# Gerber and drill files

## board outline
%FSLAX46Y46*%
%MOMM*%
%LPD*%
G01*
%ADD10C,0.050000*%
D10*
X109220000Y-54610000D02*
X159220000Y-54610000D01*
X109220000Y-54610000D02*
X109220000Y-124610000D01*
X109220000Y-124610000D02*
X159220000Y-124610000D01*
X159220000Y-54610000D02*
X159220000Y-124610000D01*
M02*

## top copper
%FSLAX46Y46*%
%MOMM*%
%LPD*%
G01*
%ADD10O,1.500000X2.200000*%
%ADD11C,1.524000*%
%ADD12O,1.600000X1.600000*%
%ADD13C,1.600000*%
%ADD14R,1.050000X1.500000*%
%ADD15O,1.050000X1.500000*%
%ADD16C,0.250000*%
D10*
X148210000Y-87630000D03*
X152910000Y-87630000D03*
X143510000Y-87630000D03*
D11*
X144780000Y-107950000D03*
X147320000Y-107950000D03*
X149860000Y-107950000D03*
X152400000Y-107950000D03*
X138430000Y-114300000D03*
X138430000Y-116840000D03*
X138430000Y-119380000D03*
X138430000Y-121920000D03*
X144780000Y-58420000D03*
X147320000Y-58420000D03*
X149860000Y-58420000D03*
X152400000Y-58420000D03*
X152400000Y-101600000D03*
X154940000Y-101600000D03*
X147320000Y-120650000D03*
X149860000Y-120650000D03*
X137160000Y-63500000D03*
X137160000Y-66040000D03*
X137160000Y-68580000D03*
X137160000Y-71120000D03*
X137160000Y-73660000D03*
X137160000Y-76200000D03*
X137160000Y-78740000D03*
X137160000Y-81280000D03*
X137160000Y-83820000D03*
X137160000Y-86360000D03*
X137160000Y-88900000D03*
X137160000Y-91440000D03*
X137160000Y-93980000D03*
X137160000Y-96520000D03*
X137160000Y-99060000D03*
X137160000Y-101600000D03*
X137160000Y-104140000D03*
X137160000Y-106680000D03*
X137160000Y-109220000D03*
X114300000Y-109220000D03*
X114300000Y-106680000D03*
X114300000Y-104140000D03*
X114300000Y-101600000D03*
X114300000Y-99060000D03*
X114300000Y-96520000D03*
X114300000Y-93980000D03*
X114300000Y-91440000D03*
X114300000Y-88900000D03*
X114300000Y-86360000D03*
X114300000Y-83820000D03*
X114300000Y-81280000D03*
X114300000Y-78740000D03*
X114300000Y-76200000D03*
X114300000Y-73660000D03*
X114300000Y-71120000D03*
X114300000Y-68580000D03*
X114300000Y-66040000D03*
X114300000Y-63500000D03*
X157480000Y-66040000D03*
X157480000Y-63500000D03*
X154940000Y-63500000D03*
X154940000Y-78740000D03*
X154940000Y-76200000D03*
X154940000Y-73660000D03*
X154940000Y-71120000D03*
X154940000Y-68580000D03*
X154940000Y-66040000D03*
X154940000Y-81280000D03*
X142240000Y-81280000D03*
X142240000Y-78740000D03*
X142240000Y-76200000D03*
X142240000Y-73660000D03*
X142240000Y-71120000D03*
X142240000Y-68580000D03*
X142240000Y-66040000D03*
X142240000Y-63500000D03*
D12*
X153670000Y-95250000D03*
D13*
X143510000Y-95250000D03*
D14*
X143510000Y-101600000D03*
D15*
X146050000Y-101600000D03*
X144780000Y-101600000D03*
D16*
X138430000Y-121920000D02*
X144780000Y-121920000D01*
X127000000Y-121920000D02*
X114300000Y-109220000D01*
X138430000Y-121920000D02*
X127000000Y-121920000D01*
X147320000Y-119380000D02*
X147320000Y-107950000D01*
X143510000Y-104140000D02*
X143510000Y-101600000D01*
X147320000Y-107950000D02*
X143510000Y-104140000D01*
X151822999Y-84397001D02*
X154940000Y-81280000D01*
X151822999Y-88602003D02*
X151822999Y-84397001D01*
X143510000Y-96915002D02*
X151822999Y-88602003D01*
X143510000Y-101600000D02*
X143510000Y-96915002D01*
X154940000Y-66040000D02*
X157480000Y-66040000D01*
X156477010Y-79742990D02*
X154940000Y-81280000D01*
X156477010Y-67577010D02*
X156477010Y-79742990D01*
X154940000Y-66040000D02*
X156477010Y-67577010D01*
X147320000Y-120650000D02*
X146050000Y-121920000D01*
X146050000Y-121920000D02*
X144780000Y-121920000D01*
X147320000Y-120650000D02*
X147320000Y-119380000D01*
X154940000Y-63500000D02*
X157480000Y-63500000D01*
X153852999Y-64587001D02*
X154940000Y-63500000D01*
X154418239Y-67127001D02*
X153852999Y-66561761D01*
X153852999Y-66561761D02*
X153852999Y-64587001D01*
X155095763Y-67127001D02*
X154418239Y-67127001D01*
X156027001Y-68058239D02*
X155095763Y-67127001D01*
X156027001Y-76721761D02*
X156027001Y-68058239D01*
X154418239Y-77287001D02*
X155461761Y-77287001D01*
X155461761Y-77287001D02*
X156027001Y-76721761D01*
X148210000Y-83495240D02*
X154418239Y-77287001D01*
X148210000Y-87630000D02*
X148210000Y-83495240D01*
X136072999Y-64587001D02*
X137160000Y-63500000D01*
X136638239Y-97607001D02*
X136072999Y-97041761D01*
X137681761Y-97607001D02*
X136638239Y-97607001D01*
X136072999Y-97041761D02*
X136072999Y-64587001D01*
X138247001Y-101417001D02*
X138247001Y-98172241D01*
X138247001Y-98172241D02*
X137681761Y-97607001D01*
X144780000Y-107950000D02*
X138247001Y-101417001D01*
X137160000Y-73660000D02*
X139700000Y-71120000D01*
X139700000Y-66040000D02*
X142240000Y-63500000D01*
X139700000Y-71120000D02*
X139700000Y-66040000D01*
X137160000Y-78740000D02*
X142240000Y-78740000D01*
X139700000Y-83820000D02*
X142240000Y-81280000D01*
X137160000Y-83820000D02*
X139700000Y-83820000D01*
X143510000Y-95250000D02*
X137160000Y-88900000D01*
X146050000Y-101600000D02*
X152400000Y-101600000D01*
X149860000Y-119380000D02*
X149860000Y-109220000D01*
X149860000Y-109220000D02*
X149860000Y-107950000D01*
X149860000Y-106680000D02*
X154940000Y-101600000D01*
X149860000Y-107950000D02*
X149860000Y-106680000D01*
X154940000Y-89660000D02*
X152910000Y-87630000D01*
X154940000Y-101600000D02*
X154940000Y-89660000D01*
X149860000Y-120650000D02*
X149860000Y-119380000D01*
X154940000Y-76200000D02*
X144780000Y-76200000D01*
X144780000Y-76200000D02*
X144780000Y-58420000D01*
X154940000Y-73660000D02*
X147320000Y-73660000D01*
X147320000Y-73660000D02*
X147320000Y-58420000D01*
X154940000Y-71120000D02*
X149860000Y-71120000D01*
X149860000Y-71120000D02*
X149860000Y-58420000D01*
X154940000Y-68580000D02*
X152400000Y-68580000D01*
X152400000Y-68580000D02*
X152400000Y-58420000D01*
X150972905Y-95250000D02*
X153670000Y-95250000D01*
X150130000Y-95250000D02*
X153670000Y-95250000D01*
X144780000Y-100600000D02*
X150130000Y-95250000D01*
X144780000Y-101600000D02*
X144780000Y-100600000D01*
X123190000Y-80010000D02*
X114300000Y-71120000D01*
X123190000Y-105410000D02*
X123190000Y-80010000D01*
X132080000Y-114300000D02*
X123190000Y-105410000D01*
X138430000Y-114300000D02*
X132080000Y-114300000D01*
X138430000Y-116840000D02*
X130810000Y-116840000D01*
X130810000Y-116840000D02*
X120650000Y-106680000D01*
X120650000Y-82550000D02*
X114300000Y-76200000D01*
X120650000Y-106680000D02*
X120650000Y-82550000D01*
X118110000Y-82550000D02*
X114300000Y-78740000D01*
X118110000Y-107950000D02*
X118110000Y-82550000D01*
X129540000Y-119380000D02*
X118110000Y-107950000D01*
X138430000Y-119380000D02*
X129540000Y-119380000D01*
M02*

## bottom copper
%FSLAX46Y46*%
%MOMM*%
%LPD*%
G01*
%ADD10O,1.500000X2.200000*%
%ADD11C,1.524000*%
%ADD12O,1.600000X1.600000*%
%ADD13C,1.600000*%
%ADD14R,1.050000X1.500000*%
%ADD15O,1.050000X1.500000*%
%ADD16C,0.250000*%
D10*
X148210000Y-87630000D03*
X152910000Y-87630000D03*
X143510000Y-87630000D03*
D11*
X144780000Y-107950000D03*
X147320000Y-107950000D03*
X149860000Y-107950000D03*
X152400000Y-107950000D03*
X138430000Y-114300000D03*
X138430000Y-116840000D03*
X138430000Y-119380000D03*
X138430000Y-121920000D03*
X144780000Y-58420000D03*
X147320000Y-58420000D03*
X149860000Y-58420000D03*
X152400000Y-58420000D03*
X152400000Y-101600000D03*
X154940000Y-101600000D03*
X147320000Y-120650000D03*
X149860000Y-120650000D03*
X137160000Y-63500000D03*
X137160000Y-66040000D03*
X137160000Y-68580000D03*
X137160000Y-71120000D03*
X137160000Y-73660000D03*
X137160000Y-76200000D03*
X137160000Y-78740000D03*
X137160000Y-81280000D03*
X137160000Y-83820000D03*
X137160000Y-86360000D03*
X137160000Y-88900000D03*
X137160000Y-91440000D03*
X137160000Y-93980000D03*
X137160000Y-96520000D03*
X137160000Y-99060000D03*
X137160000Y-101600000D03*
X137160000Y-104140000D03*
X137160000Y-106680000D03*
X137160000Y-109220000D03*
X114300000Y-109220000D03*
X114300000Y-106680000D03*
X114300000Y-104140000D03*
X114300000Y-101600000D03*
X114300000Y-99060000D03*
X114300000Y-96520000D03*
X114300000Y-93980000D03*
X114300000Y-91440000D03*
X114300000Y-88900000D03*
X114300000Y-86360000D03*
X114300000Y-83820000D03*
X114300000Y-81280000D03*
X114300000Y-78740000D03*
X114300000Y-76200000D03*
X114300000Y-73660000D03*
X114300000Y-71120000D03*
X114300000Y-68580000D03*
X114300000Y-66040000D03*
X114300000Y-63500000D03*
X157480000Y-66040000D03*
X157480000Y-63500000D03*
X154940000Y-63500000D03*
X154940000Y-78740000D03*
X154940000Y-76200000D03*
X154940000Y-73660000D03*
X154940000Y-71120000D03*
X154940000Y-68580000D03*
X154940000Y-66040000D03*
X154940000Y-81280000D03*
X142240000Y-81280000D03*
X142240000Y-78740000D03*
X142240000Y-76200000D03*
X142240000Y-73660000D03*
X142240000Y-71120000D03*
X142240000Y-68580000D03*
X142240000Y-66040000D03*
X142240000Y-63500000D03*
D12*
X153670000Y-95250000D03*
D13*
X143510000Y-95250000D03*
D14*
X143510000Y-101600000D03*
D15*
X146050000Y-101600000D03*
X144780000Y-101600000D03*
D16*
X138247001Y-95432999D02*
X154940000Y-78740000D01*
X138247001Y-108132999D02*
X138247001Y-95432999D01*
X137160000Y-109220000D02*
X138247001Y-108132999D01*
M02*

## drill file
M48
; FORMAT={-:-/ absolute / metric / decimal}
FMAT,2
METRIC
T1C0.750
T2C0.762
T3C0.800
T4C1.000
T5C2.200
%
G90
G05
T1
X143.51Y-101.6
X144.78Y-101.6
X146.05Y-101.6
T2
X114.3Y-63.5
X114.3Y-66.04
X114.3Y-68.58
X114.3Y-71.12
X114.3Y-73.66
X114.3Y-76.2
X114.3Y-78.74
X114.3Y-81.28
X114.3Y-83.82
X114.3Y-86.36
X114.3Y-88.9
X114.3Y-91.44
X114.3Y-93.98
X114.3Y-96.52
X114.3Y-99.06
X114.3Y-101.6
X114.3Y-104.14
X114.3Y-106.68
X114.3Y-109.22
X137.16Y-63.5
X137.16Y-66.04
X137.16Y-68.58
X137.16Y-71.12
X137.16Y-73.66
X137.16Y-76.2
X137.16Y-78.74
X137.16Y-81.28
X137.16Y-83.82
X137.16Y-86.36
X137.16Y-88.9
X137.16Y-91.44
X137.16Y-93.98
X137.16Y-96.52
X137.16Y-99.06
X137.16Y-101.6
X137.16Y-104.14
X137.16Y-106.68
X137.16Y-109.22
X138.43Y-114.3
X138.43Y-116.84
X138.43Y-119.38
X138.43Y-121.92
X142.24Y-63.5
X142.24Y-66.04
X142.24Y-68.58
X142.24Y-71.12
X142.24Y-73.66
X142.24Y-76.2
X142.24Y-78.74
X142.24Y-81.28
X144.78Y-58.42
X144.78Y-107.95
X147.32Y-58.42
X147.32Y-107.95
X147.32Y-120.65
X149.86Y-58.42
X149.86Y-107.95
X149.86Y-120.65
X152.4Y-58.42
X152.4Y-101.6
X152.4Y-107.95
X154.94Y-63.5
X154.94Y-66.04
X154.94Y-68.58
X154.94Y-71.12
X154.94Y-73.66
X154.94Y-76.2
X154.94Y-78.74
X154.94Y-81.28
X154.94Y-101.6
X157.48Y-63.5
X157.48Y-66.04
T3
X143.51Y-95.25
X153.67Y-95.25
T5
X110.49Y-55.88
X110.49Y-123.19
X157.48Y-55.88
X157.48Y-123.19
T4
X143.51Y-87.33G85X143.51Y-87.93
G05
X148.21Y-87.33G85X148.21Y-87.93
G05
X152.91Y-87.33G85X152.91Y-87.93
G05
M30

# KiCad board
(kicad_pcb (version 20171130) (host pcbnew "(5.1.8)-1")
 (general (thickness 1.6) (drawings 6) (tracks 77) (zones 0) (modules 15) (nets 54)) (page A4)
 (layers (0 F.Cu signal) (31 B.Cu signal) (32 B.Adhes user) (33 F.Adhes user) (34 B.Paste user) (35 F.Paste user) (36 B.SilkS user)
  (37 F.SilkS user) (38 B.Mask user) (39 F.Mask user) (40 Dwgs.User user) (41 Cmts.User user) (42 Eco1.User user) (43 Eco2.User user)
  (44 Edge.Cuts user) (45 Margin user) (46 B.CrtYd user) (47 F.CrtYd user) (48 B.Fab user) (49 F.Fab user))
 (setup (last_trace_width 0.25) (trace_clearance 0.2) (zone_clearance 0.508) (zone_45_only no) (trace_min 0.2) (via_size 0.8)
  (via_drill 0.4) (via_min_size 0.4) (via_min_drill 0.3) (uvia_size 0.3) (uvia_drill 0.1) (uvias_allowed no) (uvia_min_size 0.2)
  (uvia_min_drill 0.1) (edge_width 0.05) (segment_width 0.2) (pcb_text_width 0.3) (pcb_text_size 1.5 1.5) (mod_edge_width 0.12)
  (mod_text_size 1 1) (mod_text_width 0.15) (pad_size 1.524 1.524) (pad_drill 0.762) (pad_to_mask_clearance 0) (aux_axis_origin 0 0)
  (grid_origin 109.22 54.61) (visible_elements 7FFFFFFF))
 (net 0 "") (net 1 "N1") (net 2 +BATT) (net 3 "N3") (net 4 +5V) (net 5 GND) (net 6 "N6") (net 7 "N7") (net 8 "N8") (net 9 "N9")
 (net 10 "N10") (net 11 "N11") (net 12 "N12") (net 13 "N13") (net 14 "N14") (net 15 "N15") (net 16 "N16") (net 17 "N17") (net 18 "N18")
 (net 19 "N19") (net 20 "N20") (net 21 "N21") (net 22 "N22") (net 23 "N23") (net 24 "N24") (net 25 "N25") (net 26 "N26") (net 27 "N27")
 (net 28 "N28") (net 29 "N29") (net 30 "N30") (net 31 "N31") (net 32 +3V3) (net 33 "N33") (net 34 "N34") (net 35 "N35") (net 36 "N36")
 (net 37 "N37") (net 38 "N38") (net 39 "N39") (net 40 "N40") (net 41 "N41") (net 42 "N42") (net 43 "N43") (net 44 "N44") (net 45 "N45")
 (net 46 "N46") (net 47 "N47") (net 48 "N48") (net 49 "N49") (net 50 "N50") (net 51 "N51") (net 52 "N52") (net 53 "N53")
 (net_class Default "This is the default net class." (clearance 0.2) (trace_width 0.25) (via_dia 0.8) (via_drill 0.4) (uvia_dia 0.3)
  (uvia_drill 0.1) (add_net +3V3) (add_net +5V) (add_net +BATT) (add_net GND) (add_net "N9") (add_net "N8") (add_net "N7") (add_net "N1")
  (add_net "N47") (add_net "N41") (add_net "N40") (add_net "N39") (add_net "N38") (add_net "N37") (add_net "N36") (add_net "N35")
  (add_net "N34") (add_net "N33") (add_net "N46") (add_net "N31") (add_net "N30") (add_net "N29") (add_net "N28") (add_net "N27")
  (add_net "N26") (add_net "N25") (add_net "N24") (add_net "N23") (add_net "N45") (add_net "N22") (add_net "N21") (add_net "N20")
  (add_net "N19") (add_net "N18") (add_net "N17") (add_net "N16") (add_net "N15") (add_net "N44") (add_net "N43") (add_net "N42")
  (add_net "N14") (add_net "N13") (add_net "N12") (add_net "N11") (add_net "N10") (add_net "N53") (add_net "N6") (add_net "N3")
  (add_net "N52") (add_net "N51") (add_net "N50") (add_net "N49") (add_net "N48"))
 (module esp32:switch (layer F.Cu) (at 143.51 87.63)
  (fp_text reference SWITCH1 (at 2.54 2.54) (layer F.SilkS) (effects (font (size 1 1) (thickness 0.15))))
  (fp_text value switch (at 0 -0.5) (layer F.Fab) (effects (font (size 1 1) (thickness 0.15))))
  (pad 2 thru_hole oval (at 4.7 0) (size 1.5 2.2) (drill oval 1 1.6) (layers *.Cu *.Mask) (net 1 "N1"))
  (pad 3 thru_hole oval (at 9.4 0) (size 1.5 2.2) (drill oval 1 1.6) (layers *.Cu *.Mask) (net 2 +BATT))
  (pad 1 thru_hole oval (at 0 0) (size 1.5 2.2) (drill oval 1 1.6) (layers *.Cu *.Mask) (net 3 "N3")))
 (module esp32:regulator (layer F.Cu) (at 142.24 105.41)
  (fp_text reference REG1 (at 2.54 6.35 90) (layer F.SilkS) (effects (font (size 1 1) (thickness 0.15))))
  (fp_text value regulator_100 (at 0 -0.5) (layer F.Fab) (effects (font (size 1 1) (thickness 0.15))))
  (pad 1 thru_hole circle (at 2.54 2.54 270) (size 1.524 1.524) (drill 0.762) (layers *.Cu *.Mask) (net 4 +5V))
  (pad 2 thru_hole circle (at 5.08 2.54 270) (size 1.524 1.524) (drill 0.762) (layers *.Cu *.Mask) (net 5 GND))
  (pad 3 thru_hole circle (at 7.62 2.54 270) (size 1.524 1.524) (drill 0.762) (layers *.Cu *.Mask) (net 2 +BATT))
  (pad 4 thru_hole circle (at 10.16 2.54 270) (size 1.524 1.524) (drill 0.762) (layers *.Cu *.Mask) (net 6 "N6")))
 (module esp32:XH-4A (layer F.Cu) (at 138.43 121.92 90)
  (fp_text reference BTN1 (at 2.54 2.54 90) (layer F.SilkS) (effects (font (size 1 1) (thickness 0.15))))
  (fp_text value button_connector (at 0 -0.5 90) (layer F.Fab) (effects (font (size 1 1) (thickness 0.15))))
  (pad 4 thru_hole circle (at 7.62 0 90) (size 1.524 1.524) (drill 0.762) (layers *.Cu *.Mask) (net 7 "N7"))
  (pad 3 thru_hole circle (at 5.08 0 90) (size 1.524 1.524) (drill 0.762) (layers *.Cu *.Mask) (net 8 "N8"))
  (pad 2 thru_hole circle (at 2.54 0 90) (size 1.524 1.524) (drill 0.762) (layers *.Cu *.Mask) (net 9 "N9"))
  (pad 1 thru_hole circle (at 0 0 90) (size 1.524 1.524) (drill 0.762) (layers *.Cu *.Mask) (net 5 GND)))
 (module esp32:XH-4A (layer F.Cu) (at 152.4 58.42 180)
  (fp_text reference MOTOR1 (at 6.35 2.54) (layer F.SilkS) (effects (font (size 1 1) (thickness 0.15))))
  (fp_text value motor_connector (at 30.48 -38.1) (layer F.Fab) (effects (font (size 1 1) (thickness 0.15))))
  (pad 4 thru_hole circle (at 7.62 0 180) (size 1.524 1.524) (drill 0.762) (layers *.Cu *.Mask) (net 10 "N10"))
  (pad 3 thru_hole circle (at 5.08 0 180) (size 1.524 1.524) (drill 0.762) (layers *.Cu *.Mask) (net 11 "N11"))
  (pad 2 thru_hole circle (at 2.54 0 180) (size 1.524 1.524) (drill 0.762) (layers *.Cu *.Mask) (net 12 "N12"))
  (pad 1 thru_hole circle (at 0 0 180) (size 1.524 1.524) (drill 0.762) (layers *.Cu *.Mask) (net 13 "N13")))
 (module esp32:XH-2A (layer F.Cu) (at 154.94 101.6 180)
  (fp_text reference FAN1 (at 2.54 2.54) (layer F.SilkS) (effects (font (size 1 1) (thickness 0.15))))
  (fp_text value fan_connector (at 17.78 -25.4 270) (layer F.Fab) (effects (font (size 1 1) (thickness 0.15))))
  (pad 2 thru_hole circle (at 2.54 0 180) (size 1.524 1.524) (drill 0.762) (layers *.Cu *.Mask) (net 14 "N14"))
  (pad 1 thru_hole circle (at 0 0 180) (size 1.524 1.524) (drill 0.762) (layers *.Cu *.Mask) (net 2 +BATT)))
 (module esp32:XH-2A (layer F.Cu) (at 149.86 120.65 180)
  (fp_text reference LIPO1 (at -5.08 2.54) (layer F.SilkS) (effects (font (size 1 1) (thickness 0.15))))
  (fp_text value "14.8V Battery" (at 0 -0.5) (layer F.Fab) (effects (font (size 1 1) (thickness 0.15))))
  (pad 2 thru_hole circle (at 2.54 0 180) (size 1.524 1.524) (drill 0.762) (layers *.Cu *.Mask) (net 5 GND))
  (pad 1 thru_hole circle (at 0 0 180) (size 1.524 1.524) (drill 0.762) (layers *.Cu *.Mask) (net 2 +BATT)))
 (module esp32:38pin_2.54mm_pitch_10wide (layer F.Cu) (at 111.76 58.42)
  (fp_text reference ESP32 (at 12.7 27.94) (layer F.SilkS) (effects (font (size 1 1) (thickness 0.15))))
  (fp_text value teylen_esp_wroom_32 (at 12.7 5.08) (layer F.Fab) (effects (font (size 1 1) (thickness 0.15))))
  (pad 38 thru_hole circle (at 25.4 5.08) (size 1.524 1.524) (drill 0.762) (layers *.Cu *.Mask) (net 4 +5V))
  (pad 37 thru_hole circle (at 25.4 7.62) (size 1.524 1.524) (drill 0.762) (layers *.Cu *.Mask) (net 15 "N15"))
  (pad 36 thru_hole circle (at 25.4 10.16) (size 1.524 1.524) (drill 0.762) (layers *.Cu *.Mask) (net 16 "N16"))
  (pad 35 thru_hole circle (at 25.4 12.7) (size 1.524 1.524) (drill 0.762) (layers *.Cu *.Mask) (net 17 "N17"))
  (pad 34 thru_hole circle (at 25.4 15.24) (size 1.524 1.524) (drill 0.762) (layers *.Cu *.Mask) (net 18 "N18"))
  (pad 33 thru_hole circle (at 25.4 17.78) (size 1.524 1.524) (drill 0.762) (layers *.Cu *.Mask) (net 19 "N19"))
  (pad 32 thru_hole circle (at 25.4 20.32) (size 1.524 1.524) (drill 0.762) (layers *.Cu *.Mask) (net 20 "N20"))
  (pad 31 thru_hole circle (at 25.4 22.86) (size 1.524 1.524) (drill 0.762) (layers *.Cu *.Mask) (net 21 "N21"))
  (pad 30 thru_hole circle (at 25.4 25.4) (size 1.524 1.524) (drill 0.762) (layers *.Cu *.Mask) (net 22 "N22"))
  (pad 29 thru_hole circle (at 25.4 27.94) (size 1.524 1.524) (drill 0.762) (layers *.Cu *.Mask) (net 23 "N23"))
  (pad 28 thru_hole circle (at 25.4 30.48) (size 1.524 1.524) (drill 0.762) (layers *.Cu *.Mask) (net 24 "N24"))
  (pad 27 thru_hole circle (at 25.4 33.02) (size 1.524 1.524) (drill 0.762) (layers *.Cu *.Mask) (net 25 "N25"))
  (pad 26 thru_hole circle (at 25.4 35.56) (size 1.524 1.524) (drill 0.762) (layers *.Cu *.Mask) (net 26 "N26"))
  (pad 25 thru_hole circle (at 25.4 38.1) (size 1.524 1.524) (drill 0.762) (layers *.Cu *.Mask) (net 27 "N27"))
  (pad 24 thru_hole circle (at 25.4 40.64) (size 1.524 1.524) (drill 0.762) (layers *.Cu *.Mask) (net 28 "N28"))
  (pad 23 thru_hole circle (at 25.4 43.18) (size 1.524 1.524) (drill 0.762) (layers *.Cu *.Mask) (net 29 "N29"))
  (pad 22 thru_hole circle (at 25.4 45.72) (size 1.524 1.524) (drill 0.762) (layers *.Cu *.Mask) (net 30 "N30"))
  (pad 21 thru_hole circle (at 25.4 48.26) (size 1.524 1.524) (drill 0.762) (layers *.Cu *.Mask) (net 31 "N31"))
  (pad 20 thru_hole circle (at 25.4 50.8) (size 1.524 1.524) (drill 0.762) (layers *.Cu *.Mask) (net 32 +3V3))
  (pad 19 thru_hole circle (at 2.54 50.8) (size 1.524 1.524) (drill 0.762) (layers *.Cu *.Mask) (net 5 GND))
  (pad 18 thru_hole circle (at 2.54 48.26) (size 1.524 1.524) (drill 0.762) (layers *.Cu *.Mask) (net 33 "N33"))
  (pad 17 thru_hole circle (at 2.54 45.72) (size 1.524 1.524) (drill 0.762) (layers *.Cu *.Mask) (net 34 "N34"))
  (pad 16 thru_hole circle (at 2.54 43.18) (size 1.524 1.524) (drill 0.762) (layers *.Cu *.Mask) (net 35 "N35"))
  (pad 15 thru_hole circle (at 2.54 40.64) (size 1.524 1.524) (drill 0.762) (layers *.Cu *.Mask) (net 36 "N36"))
  (pad 14 thru_hole circle (at 2.54 38.1) (size 1.524 1.524) (drill 0.762) (layers *.Cu *.Mask) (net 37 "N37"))
  (pad 13 thru_hole circle (at 2.54 35.56) (size 1.524 1.524) (drill 0.762) (layers *.Cu *.Mask) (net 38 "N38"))
  (pad 12 thru_hole circle (at 2.54 33.02) (size 1.524 1.524) (drill 0.762) (layers *.Cu *.Mask) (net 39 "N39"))
  (pad 11 thru_hole circle (at 2.54 30.48) (size 1.524 1.524) (drill 0.762) (layers *.Cu *.Mask) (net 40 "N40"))
  (pad 10 thru_hole circle (at 2.54 27.94) (size 1.524 1.524) (drill 0.762) (layers *.Cu *.Mask) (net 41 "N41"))
  (pad 9 thru_hole circle (at 2.54 25.4) (size 1.524 1.524) (drill 0.762) (layers *.Cu *.Mask) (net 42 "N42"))
  (pad 8 thru_hole circle (at 2.54 22.86) (size 1.524 1.524) (drill 0.762) (layers *.Cu *.Mask) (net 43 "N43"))
  (pad 7 thru_hole circle (at 2.54 20.32) (size 1.524 1.524) (drill 0.762) (layers *.Cu *.Mask) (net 9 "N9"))
  (pad 6 thru_hole circle (at 2.54 17.78) (size 1.524 1.524) (drill 0.762) (layers *.Cu *.Mask) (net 8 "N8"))
  (pad 5 thru_hole circle (at 2.54 15.24) (size 1.524 1.524) (drill 0.762) (layers *.Cu *.Mask) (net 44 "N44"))
  (pad 4 thru_hole circle (at 2.54 12.7) (size 1.524 1.524) (drill 0.762) (layers *.Cu *.Mask) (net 7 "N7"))
  (pad 3 thru_hole circle (at 2.54 10.16) (size 1.524 1.524) (drill 0.762) (layers *.Cu *.Mask) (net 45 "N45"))
  (pad 2 thru_hole circle (at 2.54 7.62) (size 1.524 1.524) (drill 0.762) (layers *.Cu *.Mask) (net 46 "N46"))
  (pad 1 thru_hole circle (at 2.54 5.08) (size 1.524 1.524) (drill 0.762) (layers *.Cu *.Mask) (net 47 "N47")))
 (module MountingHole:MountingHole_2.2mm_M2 (layer F.Cu) (at 157.48 123.19)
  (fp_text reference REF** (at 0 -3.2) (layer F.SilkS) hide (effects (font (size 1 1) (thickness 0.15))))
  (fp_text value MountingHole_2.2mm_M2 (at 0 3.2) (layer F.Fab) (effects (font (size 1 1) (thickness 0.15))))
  (pad 1 np_thru_hole circle (at 0 0) (size 2.2 2.2) (drill 2.2) (layers *.Cu *.Mask)))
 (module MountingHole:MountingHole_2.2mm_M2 (layer F.Cu) (at 110.49 123.19)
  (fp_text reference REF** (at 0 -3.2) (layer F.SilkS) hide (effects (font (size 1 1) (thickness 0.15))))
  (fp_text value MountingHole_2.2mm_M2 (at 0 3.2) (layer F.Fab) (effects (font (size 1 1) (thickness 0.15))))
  (pad 1 np_thru_hole circle (at 0 0) (size 2.2 2.2) (drill 2.2) (layers *.Cu *.Mask)))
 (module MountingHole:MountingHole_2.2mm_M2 (layer F.Cu) (at 157.48 55.88)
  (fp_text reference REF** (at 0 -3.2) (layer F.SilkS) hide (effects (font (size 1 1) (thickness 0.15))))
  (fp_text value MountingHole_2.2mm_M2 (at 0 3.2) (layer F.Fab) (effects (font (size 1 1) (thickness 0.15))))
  (pad 1 np_thru_hole circle (at 0 0) (size 2.2 2.2) (drill 2.2) (layers *.Cu *.Mask)))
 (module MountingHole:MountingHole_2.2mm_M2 (layer F.Cu) (at 110.49 55.88)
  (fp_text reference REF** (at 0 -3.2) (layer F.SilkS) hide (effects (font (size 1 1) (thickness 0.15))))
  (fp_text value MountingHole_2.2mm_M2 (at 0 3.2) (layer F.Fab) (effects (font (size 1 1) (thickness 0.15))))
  (pad 1 np_thru_hole circle (at 0 0) (size 2.2 2.2) (drill 2.2) (layers *.Cu *.Mask)))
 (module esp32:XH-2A (layer F.Cu) (at 162.56 60.96 270)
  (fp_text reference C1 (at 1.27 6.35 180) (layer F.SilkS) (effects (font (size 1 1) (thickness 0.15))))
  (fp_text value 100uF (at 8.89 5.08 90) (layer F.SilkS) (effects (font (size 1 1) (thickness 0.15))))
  (pad 2 thru_hole circle (at 5.08 5.08 270) (size 1.524 1.524) (drill 0.762) (layers *.Cu *.Mask) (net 5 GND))
  (pad 1 thru_hole circle (at 2.54 5.08 270) (size 1.524 1.524) (drill 0.762) (layers *.Cu *.Mask) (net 1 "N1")))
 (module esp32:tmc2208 (layer F.Cu) (at 139.7 60.96)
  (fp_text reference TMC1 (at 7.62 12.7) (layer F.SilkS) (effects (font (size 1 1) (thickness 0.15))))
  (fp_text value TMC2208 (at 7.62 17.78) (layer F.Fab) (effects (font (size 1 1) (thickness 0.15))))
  (pad 16 thru_hole circle (at 15.24 2.54) (size 1.524 1.524) (drill 0.762) (layers *.Cu *.Mask) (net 1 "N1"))
  (pad 10 thru_hole circle (at 15.24 17.78) (size 1.524 1.524) (drill 0.762) (layers *.Cu *.Mask) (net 32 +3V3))
  (pad 11 thru_hole circle (at 15.24 15.24) (size 1.524 1.524) (drill 0.762) (layers *.Cu *.Mask) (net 10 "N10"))
  (pad 12 thru_hole circle (at 15.24 12.7) (size 1.524 1.524) (drill 0.762) (layers *.Cu *.Mask) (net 11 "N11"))
  (pad 13 thru_hole circle (at 15.24 10.16) (size 1.524 1.524) (drill 0.762) (layers *.Cu *.Mask) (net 12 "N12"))
  (pad 14 thru_hole circle (at 15.24 7.62) (size 1.524 1.524) (drill 0.762) (layers *.Cu *.Mask) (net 13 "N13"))
  (pad 15 thru_hole circle (at 15.24 5.08) (size 1.524 1.524) (drill 0.762) (layers *.Cu *.Mask) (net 5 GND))
  (pad 9 thru_hole circle (at 15.24 20.32) (size 1.524 1.524) (drill 0.762) (layers *.Cu *.Mask) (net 5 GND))
  (pad 8 thru_hole circle (at 2.54 20.32) (size 1.524 1.524) (drill 0.762) (layers *.Cu *.Mask) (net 22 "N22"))
  (pad 7 thru_hole circle (at 2.54 17.78) (size 1.524 1.524) (drill 0.762) (layers *.Cu *.Mask) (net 20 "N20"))
  (pad 6 thru_hole circle (at 2.54 15.24) (size 1.524 1.524) (drill 0.762) (layers *.Cu *.Mask) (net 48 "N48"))
  (pad 5 thru_hole circle (at 2.54 12.7) (size 1.524 1.524) (drill 0.762) (layers *.Cu *.Mask) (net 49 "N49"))
  (pad 4 thru_hole circle (at 2.54 10.16) (size 1.524 1.524) (drill 0.762) (layers *.Cu *.Mask) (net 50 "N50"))
  (pad 3 thru_hole circle (at 2.54 7.62) (size 1.524 1.524) (drill 0.762) (layers *.Cu *.Mask) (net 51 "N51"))
  (pad 2 thru_hole circle (at 2.54 5.08) (size 1.524 1.524) (drill 0.762) (layers *.Cu *.Mask) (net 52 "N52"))
  (pad 1 thru_hole circle (at 2.54 2.54) (size 1.524 1.524) (drill 0.762) (layers *.Cu *.Mask) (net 18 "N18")))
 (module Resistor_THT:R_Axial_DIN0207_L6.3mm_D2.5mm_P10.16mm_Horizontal (layer F.Cu) (at 143.51 95.25)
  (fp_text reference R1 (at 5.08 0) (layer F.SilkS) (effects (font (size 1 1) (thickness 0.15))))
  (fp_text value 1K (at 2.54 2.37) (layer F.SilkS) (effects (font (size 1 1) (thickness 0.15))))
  (pad 2 thru_hole oval (at 10.16 0) (size 1.6 1.6) (drill 0.8) (layers *.Cu *.Mask) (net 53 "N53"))
  (pad 1 thru_hole circle (at 0 0) (size 1.6 1.6) (drill 0.8) (layers *.Cu *.Mask) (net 24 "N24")))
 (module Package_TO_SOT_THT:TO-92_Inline (layer F.Cu) (at 143.51 101.6)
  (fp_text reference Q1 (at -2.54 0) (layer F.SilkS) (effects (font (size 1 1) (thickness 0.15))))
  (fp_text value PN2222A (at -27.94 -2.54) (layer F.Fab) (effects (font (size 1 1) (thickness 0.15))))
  (pad 1 thru_hole rect (at 0 0) (size 1.05 1.5) (drill 0.75) (layers *.Cu *.Mask) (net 5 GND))
  (pad 3 thru_hole oval (at 2.54 0) (size 1.05 1.5) (drill 0.75) (layers *.Cu *.Mask) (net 14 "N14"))
  (pad 2 thru_hole oval (at 1.27 0) (size 1.05 1.5) (drill 0.75) (layers *.Cu *.Mask) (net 53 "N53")))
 (gr_line (start 109.22 54.61) (end 159.22 54.61) (layer Edge.Cuts) (width 0.05))
 (gr_line (start 109.22 54.61) (end 109.22 124.61) (layer Edge.Cuts) (width 0.05))
 (gr_line (start 109.22 124.61) (end 159.22 124.61) (layer Edge.Cuts) (width 0.05))
 (gr_line (start 159.22 54.61) (end 159.22 124.61) (layer Edge.Cuts) (width 0.05))
 (segment (start 138.43 121.92) (end 144.78 121.92) (width 0.25) (layer F.Cu) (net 5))
 (segment (start 127 121.92) (end 114.3 109.22) (width 0.25) (layer F.Cu) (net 5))
 (segment (start 138.43 121.92) (end 127 121.92) (width 0.25) (layer F.Cu) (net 5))
 (segment (start 147.32 119.38) (end 147.32 107.95) (width 0.25) (layer F.Cu) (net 5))
 (segment (start 143.51 104.14) (end 143.51 101.6) (width 0.25) (layer F.Cu) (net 5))
 (segment (start 147.32 107.95) (end 143.51 104.14) (width 0.25) (layer F.Cu) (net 5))
 (segment (start 151.822999 84.397001) (end 154.94 81.28) (width 0.25) (layer F.Cu) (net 5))
 (segment (start 151.822999 88.602003) (end 151.822999 84.397001) (width 0.25) (layer F.Cu) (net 5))
 (segment (start 143.51 96.915002) (end 151.822999 88.602003) (width 0.25) (layer F.Cu) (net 5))
 (segment (start 143.51 101.6) (end 143.51 96.915002) (width 0.25) (layer F.Cu) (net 5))
 (segment (start 154.94 66.04) (end 157.48 66.04) (width 0.25) (layer F.Cu) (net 5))
 (segment (start 156.47701 79.74299) (end 154.94 81.28) (width 0.25) (layer F.Cu) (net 5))
 (segment (start 156.47701 67.57701) (end 156.47701 79.74299) (width 0.25) (layer F.Cu) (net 5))
 (segment (start 154.94 66.04) (end 156.47701 67.57701) (width 0.25) (layer F.Cu) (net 5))
 (segment (start 147.32 120.65) (end 146.05 121.92) (width 0.25) (layer F.Cu) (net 5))
 (segment (start 146.05 121.92) (end 144.78 121.92) (width 0.25) (layer F.Cu) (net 5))
 (segment (start 147.32 120.65) (end 147.32 119.38) (width 0.25) (layer F.Cu) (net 5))
 (segment (start 154.94 63.5) (end 157.48 63.5) (width 0.25) (layer F.Cu) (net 1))
 (segment (start 153.852999 64.587001) (end 154.94 63.5) (width 0.25) (layer F.Cu) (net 1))
 (segment (start 154.418239 67.127001) (end 153.852999 66.561761) (width 0.25) (layer F.Cu) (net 1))
 (segment (start 153.852999 66.561761) (end 153.852999 64.587001) (width 0.25) (layer F.Cu) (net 1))
 (segment (start 155.095763 67.127001) (end 154.418239 67.127001) (width 0.25) (layer F.Cu) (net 1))
 (segment (start 156.027001 68.058239) (end 155.095763 67.127001) (width 0.25) (layer F.Cu) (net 1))
 (segment (start 156.027001 76.721761) (end 156.027001 68.058239) (width 0.25) (layer F.Cu) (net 1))
 (segment (start 154.418239 77.287001) (end 155.461761 77.287001) (width 0.25) (layer F.Cu) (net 1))
 (segment (start 155.461761 77.287001) (end 156.027001 76.721761) (width 0.25) (layer F.Cu) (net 1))
 (segment (start 148.21 83.49524) (end 154.418239 77.287001) (width 0.25) (layer F.Cu) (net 1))
 (segment (start 148.21 87.63) (end 148.21 83.49524) (width 0.25) (layer F.Cu) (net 1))
 (segment (start 136.072999 64.587001) (end 137.16 63.5) (width 0.25) (layer F.Cu) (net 4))
 (segment (start 136.638239 97.607001) (end 136.072999 97.041761) (width 0.25) (layer F.Cu) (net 4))
 (segment (start 137.681761 97.607001) (end 136.638239 97.607001) (width 0.25) (layer F.Cu) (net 4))
 (segment (start 136.072999 97.041761) (end 136.072999 64.587001) (width 0.25) (layer F.Cu) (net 4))
 (segment (start 138.247001 101.417001) (end 138.247001 98.172241) (width 0.25) (layer F.Cu) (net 4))
 (segment (start 138.247001 98.172241) (end 137.681761 97.607001) (width 0.25) (layer F.Cu) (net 4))
 (segment (start 144.78 107.95) (end 138.247001 101.417001) (width 0.25) (layer F.Cu) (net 4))
 (segment (start 137.16 73.66) (end 139.7 71.12) (width 0.25) (layer F.Cu) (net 18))
 (segment (start 139.7 66.04) (end 142.24 63.5) (width 0.25) (layer F.Cu) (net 18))
 (segment (start 139.7 71.12) (end 139.7 66.04) (width 0.25) (layer F.Cu) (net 18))
 (segment (start 137.16 78.74) (end 142.24 78.74) (width 0.25) (layer F.Cu) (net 20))
 (segment (start 139.7 83.82) (end 142.24 81.28) (width 0.25) (layer F.Cu) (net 22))
 (segment (start 137.16 83.82) (end 139.7 83.82) (width 0.25) (layer F.Cu) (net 22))
 (segment (start 143.51 95.25) (end 137.16 88.9) (width 0.25) (layer F.Cu) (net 24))
 (segment (start 138.247001 95.432999) (end 154.94 78.74) (width 0.25) (layer B.Cu) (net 32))
 (segment (start 138.247001 108.132999) (end 138.247001 95.432999) (width 0.25) (layer B.Cu) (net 32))
 (segment (start 137.16 109.22) (end 138.247001 108.132999) (width 0.25) (layer B.Cu) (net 32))
 (segment (start 146.05 101.6) (end 152.4 101.6) (width 0.25) (layer F.Cu) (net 14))
 (segment (start 149.86 119.38) (end 149.86 109.22) (width 0.25) (layer F.Cu) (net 2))
 (segment (start 149.86 109.22) (end 149.86 107.95) (width 0.25) (layer F.Cu) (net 2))
 (segment (start 149.86 106.68) (end 154.94 101.6) (width 0.25) (layer F.Cu) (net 2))
 (segment (start 149.86 107.95) (end 149.86 106.68) (width 0.25) (layer F.Cu) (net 2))
 (segment (start 154.94 89.66) (end 152.91 87.63) (width 0.25) (layer F.Cu) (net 2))
 (segment (start 154.94 101.6) (end 154.94 89.66) (width 0.25) (layer F.Cu) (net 2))
 (segment (start 149.86 120.65) (end 149.86 119.38) (width 0.25) (layer F.Cu) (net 2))
 (segment (start 154.94 76.2) (end 144.78 76.2) (width 0.25) (layer F.Cu) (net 10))
 (segment (start 144.78 76.2) (end 144.78 58.42) (width 0.25) (layer F.Cu) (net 10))
 (segment (start 154.94 73.66) (end 147.32 73.66) (width 0.25) (layer F.Cu) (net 11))
 (segment (start 147.32 73.66) (end 147.32 58.42) (width 0.25) (layer F.Cu) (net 11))
 (segment (start 154.94 71.12) (end 149.86 71.12) (width 0.25) (layer F.Cu) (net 12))
 (segment (start 149.86 71.12) (end 149.86 58.42) (width 0.25) (layer F.Cu) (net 12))
 (segment (start 154.94 68.58) (end 152.4 68.58) (width 0.25) (layer F.Cu) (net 13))
 (segment (start 152.4 68.58) (end 152.4 58.42) (width 0.25) (layer F.Cu) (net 13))
 (segment (start 150.972905 95.25) (end 153.67 95.25) (width 0.25) (layer F.Cu) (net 53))
 (segment (start 150.13 95.25) (end 153.67 95.25) (width 0.25) (layer F.Cu) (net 53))
 (segment (start 144.78 100.6) (end 150.13 95.25) (width 0.25) (layer F.Cu) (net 53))
 (segment (start 144.78 101.6) (end 144.78 100.6) (width 0.25) (layer F.Cu) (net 53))
 (segment (start 123.19 80.01) (end 114.3 71.12) (width 0.25) (layer F.Cu) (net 7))
 (segment (start 123.19 105.41) (end 123.19 80.01) (width 0.25) (layer F.Cu) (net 7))
 (segment (start 132.08 114.3) (end 123.19 105.41) (width 0.25) (layer F.Cu) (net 7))
 (segment (start 138.43 114.3) (end 132.08 114.3) (width 0.25) (layer F.Cu) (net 7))
 (segment (start 138.43 116.84) (end 130.81 116.84) (width 0.25) (layer F.Cu) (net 8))
 (segment (start 130.81 116.84) (end 120.65 106.68) (width 0.25) (layer F.Cu) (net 8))
 (segment (start 120.65 82.55) (end 114.3 76.2) (width 0.25) (layer F.Cu) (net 8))
 (segment (start 120.65 106.68) (end 120.65 82.55) (width 0.25) (layer F.Cu) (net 8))
 (segment (start 118.11 82.55) (end 114.3 78.74) (width 0.25) (layer F.Cu) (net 9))
 (segment (start 118.11 107.95) (end 118.11 82.55) (width 0.25) (layer F.Cu) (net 9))
 (segment (start 129.54 119.38) (end 118.11 107.95) (width 0.25) (layer F.Cu) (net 9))
 (segment (start 138.43 119.38) (end 129.54 119.38) (width 0.25) (layer F.Cu) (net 9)))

